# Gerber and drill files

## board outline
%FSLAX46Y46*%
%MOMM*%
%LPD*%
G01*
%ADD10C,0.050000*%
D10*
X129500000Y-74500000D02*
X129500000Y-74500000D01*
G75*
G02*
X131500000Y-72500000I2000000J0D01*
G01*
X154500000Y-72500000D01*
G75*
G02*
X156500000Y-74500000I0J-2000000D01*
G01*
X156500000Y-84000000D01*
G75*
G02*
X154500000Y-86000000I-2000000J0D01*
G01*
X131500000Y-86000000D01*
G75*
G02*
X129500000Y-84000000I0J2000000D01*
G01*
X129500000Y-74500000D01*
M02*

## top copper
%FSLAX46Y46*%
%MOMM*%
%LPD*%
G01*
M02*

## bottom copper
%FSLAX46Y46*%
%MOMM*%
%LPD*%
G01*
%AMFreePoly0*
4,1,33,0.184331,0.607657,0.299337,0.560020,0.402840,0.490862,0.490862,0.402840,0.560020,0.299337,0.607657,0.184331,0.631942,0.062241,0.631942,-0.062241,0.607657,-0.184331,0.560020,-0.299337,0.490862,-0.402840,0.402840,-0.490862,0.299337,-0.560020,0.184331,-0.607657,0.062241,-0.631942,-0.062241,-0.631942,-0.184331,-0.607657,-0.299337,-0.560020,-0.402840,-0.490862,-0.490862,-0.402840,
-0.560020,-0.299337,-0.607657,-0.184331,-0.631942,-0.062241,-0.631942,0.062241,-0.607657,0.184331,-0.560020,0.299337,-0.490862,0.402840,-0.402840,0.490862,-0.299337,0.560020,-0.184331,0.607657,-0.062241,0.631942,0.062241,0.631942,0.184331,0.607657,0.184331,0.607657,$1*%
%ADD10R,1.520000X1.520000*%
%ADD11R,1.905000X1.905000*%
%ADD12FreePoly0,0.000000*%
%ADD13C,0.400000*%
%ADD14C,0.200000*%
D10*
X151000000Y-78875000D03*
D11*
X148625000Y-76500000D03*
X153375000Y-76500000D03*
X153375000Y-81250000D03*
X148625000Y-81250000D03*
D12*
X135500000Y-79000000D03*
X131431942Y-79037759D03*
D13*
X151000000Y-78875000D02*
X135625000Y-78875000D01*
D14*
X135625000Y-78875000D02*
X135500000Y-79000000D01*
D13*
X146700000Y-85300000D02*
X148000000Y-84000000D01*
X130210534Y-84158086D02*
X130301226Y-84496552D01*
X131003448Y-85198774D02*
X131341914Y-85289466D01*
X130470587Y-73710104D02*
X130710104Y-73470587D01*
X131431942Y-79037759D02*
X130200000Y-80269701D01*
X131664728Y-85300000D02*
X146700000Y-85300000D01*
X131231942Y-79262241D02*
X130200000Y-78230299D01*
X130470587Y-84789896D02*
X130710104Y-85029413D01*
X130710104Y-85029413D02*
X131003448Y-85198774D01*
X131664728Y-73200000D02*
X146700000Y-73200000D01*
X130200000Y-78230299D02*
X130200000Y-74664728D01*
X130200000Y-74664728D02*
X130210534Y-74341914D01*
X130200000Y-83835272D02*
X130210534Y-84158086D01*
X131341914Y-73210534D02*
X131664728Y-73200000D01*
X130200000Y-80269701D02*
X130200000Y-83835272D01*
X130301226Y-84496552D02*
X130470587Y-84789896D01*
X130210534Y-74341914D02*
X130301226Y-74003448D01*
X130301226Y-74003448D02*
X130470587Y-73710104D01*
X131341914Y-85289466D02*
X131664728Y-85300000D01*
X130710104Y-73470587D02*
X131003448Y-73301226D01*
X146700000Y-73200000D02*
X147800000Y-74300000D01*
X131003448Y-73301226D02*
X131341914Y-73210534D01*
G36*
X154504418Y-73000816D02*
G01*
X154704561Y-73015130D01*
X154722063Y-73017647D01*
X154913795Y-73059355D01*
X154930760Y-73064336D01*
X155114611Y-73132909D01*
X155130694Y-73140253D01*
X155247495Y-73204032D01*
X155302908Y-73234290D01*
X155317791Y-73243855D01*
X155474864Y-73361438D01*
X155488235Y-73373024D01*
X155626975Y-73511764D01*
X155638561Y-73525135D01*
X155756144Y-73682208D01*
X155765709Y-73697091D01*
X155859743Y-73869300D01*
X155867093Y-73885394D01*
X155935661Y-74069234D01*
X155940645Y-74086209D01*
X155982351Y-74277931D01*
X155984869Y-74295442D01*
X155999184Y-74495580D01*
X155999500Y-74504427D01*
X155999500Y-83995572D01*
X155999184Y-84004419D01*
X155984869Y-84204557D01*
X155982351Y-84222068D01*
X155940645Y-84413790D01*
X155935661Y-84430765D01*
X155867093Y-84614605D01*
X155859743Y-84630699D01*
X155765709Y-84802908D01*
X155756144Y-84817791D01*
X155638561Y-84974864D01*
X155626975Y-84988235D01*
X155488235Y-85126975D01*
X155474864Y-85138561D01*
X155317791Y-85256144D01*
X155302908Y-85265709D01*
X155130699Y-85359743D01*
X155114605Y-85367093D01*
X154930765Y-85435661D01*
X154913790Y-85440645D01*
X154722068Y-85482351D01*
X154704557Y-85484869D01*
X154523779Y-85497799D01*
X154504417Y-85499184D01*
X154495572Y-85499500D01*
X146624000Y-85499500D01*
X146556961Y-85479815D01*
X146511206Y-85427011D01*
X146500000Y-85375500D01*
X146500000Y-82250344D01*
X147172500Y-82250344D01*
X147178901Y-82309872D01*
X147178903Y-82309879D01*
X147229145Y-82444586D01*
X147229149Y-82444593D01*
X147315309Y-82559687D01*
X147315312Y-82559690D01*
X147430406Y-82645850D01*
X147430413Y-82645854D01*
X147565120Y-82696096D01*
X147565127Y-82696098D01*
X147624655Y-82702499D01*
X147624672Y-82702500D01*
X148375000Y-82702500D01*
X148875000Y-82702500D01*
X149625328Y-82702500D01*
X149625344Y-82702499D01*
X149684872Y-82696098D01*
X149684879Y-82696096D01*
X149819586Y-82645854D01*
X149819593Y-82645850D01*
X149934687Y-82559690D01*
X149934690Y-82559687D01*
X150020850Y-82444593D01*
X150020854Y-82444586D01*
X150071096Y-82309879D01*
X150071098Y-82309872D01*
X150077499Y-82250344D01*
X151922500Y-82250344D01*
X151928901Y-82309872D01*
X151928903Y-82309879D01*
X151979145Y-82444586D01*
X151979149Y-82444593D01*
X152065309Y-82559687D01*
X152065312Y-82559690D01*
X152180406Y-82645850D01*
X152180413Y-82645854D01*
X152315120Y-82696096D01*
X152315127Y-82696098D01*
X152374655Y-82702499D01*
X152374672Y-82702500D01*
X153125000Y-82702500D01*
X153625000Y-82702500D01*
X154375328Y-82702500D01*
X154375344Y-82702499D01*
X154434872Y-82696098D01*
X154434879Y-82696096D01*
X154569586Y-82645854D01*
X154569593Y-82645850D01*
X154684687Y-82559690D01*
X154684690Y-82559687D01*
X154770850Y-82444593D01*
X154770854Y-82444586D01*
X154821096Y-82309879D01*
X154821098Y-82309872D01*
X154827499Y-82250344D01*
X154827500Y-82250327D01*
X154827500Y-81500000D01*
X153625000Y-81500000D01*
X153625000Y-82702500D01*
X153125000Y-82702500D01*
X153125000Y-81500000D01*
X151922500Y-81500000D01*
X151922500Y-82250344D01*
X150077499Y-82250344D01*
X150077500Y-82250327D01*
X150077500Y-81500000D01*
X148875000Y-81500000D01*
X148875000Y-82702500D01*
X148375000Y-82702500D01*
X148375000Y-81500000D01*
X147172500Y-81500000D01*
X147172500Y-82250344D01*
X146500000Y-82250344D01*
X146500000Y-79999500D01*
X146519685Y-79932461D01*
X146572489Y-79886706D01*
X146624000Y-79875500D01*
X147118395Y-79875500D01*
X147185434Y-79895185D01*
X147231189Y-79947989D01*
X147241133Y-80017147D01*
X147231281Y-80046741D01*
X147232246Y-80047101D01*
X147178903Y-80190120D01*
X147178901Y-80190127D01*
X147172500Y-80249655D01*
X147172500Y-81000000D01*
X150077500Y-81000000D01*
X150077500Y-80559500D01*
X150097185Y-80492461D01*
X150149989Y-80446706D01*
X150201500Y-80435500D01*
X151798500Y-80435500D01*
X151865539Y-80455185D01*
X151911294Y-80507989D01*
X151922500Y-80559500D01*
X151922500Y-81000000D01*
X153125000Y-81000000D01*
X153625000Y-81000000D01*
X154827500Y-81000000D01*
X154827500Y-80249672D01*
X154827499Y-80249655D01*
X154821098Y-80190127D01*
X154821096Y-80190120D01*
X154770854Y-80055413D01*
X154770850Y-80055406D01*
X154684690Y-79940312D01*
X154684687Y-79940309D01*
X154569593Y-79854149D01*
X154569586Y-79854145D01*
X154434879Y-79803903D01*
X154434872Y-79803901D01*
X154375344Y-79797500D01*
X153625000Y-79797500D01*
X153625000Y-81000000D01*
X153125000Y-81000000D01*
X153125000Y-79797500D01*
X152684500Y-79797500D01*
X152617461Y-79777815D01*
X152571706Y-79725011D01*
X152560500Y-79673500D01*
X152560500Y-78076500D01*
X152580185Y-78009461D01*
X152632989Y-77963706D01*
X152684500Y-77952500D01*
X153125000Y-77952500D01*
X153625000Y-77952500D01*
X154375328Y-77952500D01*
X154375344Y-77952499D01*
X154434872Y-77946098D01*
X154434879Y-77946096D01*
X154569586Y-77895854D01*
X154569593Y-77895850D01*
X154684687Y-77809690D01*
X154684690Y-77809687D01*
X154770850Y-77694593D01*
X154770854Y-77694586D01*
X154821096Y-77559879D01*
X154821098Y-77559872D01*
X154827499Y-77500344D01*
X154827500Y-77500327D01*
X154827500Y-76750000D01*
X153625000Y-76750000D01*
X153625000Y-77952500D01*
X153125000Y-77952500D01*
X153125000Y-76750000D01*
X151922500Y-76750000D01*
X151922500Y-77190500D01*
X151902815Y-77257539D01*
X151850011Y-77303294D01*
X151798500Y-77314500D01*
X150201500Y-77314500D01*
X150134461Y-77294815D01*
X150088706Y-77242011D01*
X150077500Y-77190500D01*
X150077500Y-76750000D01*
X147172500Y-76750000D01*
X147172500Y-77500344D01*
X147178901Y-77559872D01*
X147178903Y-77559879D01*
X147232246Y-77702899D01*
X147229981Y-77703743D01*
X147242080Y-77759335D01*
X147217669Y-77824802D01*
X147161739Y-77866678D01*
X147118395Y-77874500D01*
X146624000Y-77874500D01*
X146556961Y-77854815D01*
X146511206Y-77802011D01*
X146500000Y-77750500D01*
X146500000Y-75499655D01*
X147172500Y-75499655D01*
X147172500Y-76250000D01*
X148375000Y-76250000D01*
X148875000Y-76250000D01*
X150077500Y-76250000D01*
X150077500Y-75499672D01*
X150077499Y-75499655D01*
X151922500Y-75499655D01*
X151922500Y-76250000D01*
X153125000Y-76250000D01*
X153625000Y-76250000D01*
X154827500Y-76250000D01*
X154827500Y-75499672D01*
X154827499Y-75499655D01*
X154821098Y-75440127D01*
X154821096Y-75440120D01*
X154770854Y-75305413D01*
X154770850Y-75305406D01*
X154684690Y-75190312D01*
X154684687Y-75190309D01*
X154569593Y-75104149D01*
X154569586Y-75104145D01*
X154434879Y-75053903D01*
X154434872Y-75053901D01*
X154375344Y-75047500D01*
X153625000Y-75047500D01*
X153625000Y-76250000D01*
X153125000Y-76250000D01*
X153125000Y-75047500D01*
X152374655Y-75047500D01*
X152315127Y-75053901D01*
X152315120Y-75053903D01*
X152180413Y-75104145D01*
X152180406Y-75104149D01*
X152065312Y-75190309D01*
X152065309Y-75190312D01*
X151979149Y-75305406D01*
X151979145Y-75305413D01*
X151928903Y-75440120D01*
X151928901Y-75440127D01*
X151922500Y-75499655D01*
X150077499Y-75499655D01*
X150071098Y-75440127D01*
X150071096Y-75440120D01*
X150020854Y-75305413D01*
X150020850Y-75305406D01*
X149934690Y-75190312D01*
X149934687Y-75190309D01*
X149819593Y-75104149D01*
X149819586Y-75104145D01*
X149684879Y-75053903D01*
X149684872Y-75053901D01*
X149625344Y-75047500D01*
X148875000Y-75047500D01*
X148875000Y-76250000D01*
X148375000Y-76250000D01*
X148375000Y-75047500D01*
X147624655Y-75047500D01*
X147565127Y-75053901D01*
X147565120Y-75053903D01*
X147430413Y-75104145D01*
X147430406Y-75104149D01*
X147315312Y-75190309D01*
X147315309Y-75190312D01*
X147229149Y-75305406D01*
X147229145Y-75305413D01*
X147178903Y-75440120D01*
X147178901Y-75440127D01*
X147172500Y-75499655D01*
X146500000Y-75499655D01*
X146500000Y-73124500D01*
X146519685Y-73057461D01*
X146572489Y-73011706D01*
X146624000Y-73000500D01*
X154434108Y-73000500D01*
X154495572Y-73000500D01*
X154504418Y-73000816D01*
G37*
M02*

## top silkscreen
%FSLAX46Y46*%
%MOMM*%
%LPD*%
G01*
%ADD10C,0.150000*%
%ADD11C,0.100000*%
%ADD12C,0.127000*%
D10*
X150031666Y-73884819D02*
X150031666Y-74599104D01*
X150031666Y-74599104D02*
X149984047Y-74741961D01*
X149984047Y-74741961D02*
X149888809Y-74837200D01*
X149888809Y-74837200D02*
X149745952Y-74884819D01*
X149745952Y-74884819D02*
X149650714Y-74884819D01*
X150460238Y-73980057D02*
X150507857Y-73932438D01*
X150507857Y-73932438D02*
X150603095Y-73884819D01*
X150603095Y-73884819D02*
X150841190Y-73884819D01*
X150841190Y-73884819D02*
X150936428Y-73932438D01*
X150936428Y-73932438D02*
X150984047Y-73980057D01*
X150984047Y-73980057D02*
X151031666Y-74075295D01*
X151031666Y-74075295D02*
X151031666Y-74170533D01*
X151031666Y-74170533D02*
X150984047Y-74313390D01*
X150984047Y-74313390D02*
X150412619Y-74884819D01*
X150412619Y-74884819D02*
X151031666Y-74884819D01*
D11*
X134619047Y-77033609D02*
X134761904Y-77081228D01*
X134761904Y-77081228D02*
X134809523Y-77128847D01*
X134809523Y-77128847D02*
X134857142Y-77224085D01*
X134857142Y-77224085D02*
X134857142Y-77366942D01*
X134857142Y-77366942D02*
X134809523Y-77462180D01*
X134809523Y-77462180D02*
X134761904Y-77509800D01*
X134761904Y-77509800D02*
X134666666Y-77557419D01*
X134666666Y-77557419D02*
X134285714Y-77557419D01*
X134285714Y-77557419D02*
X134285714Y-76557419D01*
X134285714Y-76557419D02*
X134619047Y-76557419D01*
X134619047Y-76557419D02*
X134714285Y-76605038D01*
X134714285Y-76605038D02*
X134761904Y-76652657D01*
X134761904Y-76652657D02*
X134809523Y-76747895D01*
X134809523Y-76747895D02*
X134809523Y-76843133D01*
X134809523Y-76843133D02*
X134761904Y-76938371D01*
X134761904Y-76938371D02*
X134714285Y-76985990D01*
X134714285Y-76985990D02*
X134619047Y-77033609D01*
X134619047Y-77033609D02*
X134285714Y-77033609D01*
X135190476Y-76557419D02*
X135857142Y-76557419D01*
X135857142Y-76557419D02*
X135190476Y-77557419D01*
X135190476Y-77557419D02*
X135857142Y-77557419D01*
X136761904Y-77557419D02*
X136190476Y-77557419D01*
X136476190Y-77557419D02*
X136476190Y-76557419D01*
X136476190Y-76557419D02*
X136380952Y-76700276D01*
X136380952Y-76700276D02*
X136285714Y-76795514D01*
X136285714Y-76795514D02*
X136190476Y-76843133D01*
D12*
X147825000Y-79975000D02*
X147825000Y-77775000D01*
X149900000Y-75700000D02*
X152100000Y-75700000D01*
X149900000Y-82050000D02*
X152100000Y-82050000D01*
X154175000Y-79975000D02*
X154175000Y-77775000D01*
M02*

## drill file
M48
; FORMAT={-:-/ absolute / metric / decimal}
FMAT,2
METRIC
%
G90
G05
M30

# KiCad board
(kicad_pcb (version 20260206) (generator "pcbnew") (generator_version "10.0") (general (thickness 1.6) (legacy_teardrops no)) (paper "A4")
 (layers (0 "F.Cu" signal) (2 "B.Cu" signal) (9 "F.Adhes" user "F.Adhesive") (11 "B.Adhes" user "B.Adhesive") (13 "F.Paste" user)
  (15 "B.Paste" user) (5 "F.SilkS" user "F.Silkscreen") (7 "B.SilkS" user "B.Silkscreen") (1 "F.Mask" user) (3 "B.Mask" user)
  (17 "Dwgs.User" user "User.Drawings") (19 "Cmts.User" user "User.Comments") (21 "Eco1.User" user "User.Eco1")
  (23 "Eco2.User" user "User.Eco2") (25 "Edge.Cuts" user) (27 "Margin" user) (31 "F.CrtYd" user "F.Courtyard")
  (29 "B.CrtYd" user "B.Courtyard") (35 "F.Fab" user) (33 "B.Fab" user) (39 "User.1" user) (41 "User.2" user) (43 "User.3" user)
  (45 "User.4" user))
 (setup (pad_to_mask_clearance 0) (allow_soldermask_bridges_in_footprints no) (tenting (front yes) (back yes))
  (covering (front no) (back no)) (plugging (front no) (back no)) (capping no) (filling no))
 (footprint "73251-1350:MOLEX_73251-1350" (layer "F.Cu") (at 151 78.875)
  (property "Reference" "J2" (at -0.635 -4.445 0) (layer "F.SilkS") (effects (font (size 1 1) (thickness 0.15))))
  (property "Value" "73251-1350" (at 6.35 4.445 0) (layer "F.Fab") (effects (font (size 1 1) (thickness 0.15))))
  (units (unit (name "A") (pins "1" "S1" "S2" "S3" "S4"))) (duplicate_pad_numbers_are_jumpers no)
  (fp_line (start -3.175 1.1) (end -3.175 -1.1) (stroke (width 0.127) (type solid)) (layer "F.SilkS"))
  (fp_line (start -1.1 -3.175) (end 1.1 -3.175) (stroke (width 0.127) (type solid)) (layer "F.SilkS"))
  (fp_line (start -1.1 3.175) (end 1.1 3.175) (stroke (width 0.127) (type solid)) (layer "F.SilkS"))
  (fp_line (start 3.175 1.1) (end 3.175 -1.1) (stroke (width 0.127) (type solid)) (layer "F.SilkS"))
  (pad "1" smd rect (at 0 0) (size 1.52 1.52) (layers "B.Cu" "B.Mask" "B.SilkS" "B.Paste") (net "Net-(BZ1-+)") (solder_mask_margin 0.0762))
  (pad "S1" smd rect (at -2.375 -2.375) (size 1.905 1.905) (layers "B.Cu" "B.Mask" "B.SilkS" "B.Paste") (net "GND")
   (solder_mask_margin 0.0762))
  (pad "S2" smd rect (at 2.375 -2.375) (size 1.905 1.905) (layers "B.Cu" "B.Mask" "B.SilkS" "B.Paste") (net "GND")
   (solder_mask_margin 0.0762))
  (pad "S3" smd rect (at 2.375 2.375) (size 1.905 1.905) (layers "B.Cu" "B.Mask" "B.SilkS" "B.Paste") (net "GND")
   (solder_mask_margin 0.0762))
  (pad "S4" smd rect (at -2.375 2.375) (size 1.905 1.905) (layers "B.Cu" "B.Mask" "B.SilkS" "B.Paste") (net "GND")
   (solder_mask_margin 0.0762)))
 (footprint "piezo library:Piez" (layer "F.Cu") (at 135.5 79.1)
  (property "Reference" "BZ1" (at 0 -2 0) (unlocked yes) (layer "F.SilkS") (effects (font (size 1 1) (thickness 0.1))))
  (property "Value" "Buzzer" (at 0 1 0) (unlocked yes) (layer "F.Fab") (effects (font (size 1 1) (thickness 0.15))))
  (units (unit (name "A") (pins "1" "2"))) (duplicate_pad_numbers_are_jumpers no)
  (pad "1" smd custom (at 0 -0.1) (size 1.27 1.27) (layers "B.Cu" "B.Mask" "B.SilkS" "B.Paste") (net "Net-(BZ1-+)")
   (thermal_bridge_angle 90) (options (clearance outline) (anchor circle)) (primitives))
  (pad "2" smd custom (at -4.068058 -0.062241) (size 1.27 1.27) (layers "B.Cu" "B.Mask" "B.SilkS" "B.Paste") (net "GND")
   (thermal_bridge_angle 90) (options (clearance outline) (anchor circle)) (primitives)))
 (gr_rect (start 129.5 72.5) (end 156.5 86) (radius 2) (stroke (width 0.05) (type solid)) (fill no) (layer "Edge.Cuts"))
 (segment (start 151 78.875) (end 135.625 78.875) (width 0.4) (layer "B.Cu") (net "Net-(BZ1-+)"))
 (segment (start 135.625 78.875) (end 135.5 79) (width 0.2) (layer "B.Cu") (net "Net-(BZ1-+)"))
 (segment (start 146.7 85.3) (end 148 84) (width 0.4) (layer "B.Cu") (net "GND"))
 (segment (start 130.210534 84.158086) (end 130.301226 84.496552) (width 0.4) (layer "B.Cu") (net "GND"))
 (segment (start 131.003448 85.198774) (end 131.341914 85.289466) (width 0.4) (layer "B.Cu") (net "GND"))
 (segment (start 130.470587 73.710104) (end 130.710104 73.470587) (width 0.4) (layer "B.Cu") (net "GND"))
 (segment (start 131.431942 79.037759) (end 130.2 80.269701) (width 0.4) (layer "B.Cu") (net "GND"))
 (segment (start 131.664728 85.3) (end 146.7 85.3) (width 0.4) (layer "B.Cu") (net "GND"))
 (segment (start 131.231942 79.262241) (end 130.2 78.230299) (width 0.4) (layer "B.Cu") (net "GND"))
 (segment (start 130.470587 84.789896) (end 130.710104 85.029413) (width 0.4) (layer "B.Cu") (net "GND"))
 (segment (start 130.710104 85.029413) (end 131.003448 85.198774) (width 0.4) (layer "B.Cu") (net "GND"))
 (segment (start 131.664728 73.2) (end 146.7 73.2) (width 0.4) (layer "B.Cu") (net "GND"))
 (segment (start 130.2 78.230299) (end 130.2 74.664728) (width 0.4) (layer "B.Cu") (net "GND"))
 (segment (start 130.2 74.664728) (end 130.210534 74.341914) (width 0.4) (layer "B.Cu") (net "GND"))
 (segment (start 130.2 83.835272) (end 130.210534 84.158086) (width 0.4) (layer "B.Cu") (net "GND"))
 (segment (start 131.341914 73.210534) (end 131.664728 73.2) (width 0.4) (layer "B.Cu") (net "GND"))
 (segment (start 130.2 80.269701) (end 130.2 83.835272) (width 0.4) (layer "B.Cu") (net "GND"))
 (segment (start 130.301226 84.496552) (end 130.470587 84.789896) (width 0.4) (layer "B.Cu") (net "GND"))
 (segment (start 130.210534 74.341914) (end 130.301226 74.003448) (width 0.4) (layer "B.Cu") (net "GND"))
 (segment (start 130.301226 74.003448) (end 130.470587 73.710104) (width 0.4) (layer "B.Cu") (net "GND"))
 (segment (start 131.341914 85.289466) (end 131.664728 85.3) (width 0.4) (layer "B.Cu") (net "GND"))
 (segment (start 130.710104 73.470587) (end 131.003448 73.301226) (width 0.4) (layer "B.Cu") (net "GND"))
 (segment (start 146.7 73.2) (end 147.8 74.3) (width 0.4) (layer "B.Cu") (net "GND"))
 (segment (start 131.003448 73.301226) (end 131.341914 73.210534) (width 0.4) (layer "B.Cu") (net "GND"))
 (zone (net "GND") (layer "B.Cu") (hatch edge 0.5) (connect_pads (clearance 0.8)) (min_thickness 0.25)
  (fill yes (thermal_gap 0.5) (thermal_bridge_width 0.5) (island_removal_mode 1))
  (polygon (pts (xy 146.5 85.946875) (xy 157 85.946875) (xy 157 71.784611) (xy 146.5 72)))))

